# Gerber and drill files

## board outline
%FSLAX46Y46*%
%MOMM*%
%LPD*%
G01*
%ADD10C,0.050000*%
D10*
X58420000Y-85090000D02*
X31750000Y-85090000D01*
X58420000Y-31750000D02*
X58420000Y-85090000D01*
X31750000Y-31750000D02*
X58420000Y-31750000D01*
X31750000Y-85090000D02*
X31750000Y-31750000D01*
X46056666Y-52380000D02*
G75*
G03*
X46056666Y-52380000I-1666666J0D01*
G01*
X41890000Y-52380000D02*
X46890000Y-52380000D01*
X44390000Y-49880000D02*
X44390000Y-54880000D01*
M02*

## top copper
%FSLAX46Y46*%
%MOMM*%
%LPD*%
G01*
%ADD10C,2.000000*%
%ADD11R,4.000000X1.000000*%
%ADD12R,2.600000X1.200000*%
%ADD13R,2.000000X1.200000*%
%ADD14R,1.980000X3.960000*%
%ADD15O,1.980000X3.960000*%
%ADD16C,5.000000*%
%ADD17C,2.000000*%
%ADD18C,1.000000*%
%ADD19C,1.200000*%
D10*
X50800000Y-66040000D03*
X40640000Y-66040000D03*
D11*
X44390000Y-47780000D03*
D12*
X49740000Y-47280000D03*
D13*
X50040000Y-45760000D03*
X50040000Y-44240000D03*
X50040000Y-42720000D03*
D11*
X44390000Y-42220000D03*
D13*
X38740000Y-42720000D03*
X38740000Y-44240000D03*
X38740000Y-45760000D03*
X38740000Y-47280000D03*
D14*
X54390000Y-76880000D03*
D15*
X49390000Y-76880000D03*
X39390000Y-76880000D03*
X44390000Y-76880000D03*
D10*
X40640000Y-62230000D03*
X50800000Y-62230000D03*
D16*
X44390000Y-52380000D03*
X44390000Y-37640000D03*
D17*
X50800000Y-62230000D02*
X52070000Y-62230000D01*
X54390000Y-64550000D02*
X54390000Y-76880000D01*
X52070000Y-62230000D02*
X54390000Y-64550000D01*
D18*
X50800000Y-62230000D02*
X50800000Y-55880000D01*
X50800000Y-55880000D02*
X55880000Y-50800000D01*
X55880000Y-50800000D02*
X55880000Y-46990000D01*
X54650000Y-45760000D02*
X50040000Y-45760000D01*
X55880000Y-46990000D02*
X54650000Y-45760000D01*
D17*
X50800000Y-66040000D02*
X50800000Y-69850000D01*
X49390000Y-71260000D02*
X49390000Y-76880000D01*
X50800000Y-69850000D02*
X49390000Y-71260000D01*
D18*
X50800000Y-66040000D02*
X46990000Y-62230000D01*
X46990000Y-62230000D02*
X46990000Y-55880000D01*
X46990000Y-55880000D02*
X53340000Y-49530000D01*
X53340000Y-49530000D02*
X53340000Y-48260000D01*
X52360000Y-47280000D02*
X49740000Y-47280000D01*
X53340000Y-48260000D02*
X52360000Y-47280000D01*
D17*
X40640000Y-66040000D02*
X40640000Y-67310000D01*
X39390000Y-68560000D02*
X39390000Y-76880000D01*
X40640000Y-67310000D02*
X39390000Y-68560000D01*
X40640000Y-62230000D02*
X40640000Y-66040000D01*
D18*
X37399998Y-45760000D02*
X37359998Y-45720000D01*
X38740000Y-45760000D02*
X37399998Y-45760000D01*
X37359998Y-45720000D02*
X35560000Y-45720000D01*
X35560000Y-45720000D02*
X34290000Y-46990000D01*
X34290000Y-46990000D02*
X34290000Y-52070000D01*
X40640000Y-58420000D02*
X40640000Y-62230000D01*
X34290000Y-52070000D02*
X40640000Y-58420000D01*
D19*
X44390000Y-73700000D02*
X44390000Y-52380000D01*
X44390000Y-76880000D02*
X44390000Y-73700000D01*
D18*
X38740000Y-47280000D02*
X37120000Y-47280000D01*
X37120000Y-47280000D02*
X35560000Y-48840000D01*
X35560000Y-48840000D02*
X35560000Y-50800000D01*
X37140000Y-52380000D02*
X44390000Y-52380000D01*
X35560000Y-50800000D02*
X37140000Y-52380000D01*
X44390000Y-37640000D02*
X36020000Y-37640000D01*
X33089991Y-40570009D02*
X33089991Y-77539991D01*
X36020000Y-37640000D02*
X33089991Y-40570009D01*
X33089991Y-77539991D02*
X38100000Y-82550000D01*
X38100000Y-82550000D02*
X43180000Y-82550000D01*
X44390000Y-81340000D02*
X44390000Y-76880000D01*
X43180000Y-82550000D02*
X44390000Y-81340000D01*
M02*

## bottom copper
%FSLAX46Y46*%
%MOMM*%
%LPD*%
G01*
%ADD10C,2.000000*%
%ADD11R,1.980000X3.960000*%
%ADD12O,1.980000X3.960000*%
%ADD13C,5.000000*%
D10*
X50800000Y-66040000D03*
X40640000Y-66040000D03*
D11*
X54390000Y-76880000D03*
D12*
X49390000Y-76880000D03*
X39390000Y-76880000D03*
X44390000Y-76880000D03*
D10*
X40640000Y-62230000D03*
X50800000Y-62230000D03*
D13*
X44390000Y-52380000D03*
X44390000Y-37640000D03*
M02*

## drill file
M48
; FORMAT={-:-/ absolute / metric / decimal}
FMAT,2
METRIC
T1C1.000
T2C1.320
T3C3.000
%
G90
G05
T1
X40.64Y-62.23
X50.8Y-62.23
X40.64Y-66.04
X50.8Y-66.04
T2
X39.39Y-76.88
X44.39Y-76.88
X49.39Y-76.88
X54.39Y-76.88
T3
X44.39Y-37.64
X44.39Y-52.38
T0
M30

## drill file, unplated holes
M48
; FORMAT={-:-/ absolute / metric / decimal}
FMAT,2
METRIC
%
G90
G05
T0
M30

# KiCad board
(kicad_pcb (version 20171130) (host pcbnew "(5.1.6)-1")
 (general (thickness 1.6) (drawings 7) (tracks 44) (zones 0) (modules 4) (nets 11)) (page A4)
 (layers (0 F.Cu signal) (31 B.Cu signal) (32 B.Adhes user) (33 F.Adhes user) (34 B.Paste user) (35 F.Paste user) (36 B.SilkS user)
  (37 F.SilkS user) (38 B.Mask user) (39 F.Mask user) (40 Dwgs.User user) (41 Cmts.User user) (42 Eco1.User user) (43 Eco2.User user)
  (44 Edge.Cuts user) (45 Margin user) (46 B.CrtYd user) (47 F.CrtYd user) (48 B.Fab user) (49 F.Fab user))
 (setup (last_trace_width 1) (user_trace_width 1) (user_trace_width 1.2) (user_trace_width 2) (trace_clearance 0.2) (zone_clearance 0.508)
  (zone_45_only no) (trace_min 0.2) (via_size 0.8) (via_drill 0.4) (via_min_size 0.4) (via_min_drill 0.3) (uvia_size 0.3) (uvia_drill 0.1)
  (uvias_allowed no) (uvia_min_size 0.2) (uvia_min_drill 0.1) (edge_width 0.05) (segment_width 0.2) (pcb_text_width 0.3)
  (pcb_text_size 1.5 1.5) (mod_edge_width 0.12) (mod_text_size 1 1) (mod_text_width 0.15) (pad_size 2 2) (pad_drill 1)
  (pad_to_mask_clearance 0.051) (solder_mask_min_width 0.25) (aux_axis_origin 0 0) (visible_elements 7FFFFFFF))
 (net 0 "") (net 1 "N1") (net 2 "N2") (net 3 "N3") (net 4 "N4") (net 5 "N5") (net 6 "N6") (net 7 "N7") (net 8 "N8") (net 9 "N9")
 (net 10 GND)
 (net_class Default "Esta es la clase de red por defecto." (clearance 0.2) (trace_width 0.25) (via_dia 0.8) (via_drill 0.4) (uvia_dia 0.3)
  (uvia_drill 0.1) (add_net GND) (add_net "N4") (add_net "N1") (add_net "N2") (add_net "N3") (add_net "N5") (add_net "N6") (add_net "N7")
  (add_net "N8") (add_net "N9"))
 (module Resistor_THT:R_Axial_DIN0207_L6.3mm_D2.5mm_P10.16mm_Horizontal (layer F.Cu) (at 50.8 66.04 180)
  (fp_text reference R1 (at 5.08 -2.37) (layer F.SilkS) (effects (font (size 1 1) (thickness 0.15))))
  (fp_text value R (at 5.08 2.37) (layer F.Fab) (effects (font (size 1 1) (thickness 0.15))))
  (pad 1 thru_hole circle (at 0 0 180) (size 2 2) (drill 1) (layers *.Cu *.Mask) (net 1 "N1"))
  (pad 2 thru_hole circle (at 10.16 0 180) (size 2 2) (drill 1) (layers *.Cu *.Mask) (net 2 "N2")))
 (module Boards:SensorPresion (layer F.Cu) (at 44.39 47.78)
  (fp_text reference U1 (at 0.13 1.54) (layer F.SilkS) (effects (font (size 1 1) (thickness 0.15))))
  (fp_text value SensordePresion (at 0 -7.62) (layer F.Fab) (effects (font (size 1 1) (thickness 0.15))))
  (pad 10 smd rect (at 0 0) (size 4 1) (layers F.Cu F.Paste F.Mask) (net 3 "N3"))
  (pad 1 smd rect (at 5.35 -0.5) (size 2.6 1.2) (layers F.Cu F.Paste F.Mask) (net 1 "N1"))
  (pad 2 smd rect (at 5.65 -2.02) (size 2 1.2) (layers F.Cu F.Paste F.Mask) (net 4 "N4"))
  (pad 3 smd rect (at 5.65 -3.54) (size 2 1.2) (layers F.Cu F.Paste F.Mask) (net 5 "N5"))
  (pad 4 smd rect (at 5.65 -5.06) (size 2 1.2) (layers F.Cu F.Paste F.Mask) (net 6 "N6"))
  (pad 5 smd rect (at 0 -5.56) (size 4 1) (layers F.Cu F.Paste F.Mask) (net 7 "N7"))
  (pad 6 smd rect (at -5.65 -5.06) (size 2 1.2) (layers F.Cu F.Paste F.Mask) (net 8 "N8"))
  (pad 7 smd rect (at -5.65 -3.54) (size 2 1.2) (layers F.Cu F.Paste F.Mask) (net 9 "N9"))
  (pad 8 smd rect (at -5.65 -2.02) (size 2 1.2) (layers F.Cu F.Paste F.Mask) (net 2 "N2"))
  (pad 9 smd rect (at -5.65 -0.5) (size 2 1.2) (layers F.Cu F.Paste F.Mask) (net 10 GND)))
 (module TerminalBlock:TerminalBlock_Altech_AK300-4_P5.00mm (layer F.Cu) (at 54.39 76.88 180)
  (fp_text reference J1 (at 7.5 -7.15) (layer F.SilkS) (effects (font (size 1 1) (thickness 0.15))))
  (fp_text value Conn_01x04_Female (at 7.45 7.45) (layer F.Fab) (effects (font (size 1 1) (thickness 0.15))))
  (pad 1 thru_hole rect (at 0 0 180) (size 1.98 3.96) (drill 1.32) (layers *.Cu *.Mask) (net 4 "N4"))
  (pad 2 thru_hole oval (at 5 0 180) (size 1.98 3.96) (drill 1.32) (layers *.Cu *.Mask) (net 1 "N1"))
  (pad 4 thru_hole oval (at 15 0 180) (size 1.98 3.96) (drill 1.32) (layers *.Cu *.Mask) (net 2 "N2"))
  (pad 3 thru_hole oval (at 10 0 180) (size 1.98 3.96) (drill 1.32) (layers *.Cu *.Mask) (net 10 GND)))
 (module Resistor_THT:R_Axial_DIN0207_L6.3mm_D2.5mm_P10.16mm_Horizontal (layer F.Cu) (at 50.8 62.23 180)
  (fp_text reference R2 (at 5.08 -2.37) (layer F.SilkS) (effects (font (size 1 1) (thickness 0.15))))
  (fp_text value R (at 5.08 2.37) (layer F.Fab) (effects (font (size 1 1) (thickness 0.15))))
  (pad 2 thru_hole circle (at 10.16 0 180) (size 2 2) (drill 1) (layers *.Cu *.Mask) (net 2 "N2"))
  (pad 1 thru_hole circle (at 0 0 180) (size 2 2) (drill 1) (layers *.Cu *.Mask) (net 4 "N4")))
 (gr_line (start 58.42 85.09) (end 31.75 85.09) (layer Edge.Cuts) (width 0.05))
 (gr_line (start 58.42 31.75) (end 58.42 85.09) (layer Edge.Cuts) (width 0.05))
 (gr_line (start 31.75 31.75) (end 58.42 31.75) (layer Edge.Cuts) (width 0.05))
 (gr_line (start 31.75 85.09) (end 31.75 31.75) (layer Edge.Cuts) (width 0.05))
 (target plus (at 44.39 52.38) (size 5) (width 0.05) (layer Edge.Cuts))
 (segment (start 50.8 62.23) (end 52.07 62.23) (width 2) (layer F.Cu) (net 4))
 (segment (start 54.39 64.55) (end 54.39 76.88) (width 2) (layer F.Cu) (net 4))
 (segment (start 52.07 62.23) (end 54.39 64.55) (width 2) (layer F.Cu) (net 4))
 (segment (start 50.8 62.23) (end 50.8 55.88) (width 1) (layer F.Cu) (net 4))
 (segment (start 50.8 55.88) (end 55.88 50.8) (width 1) (layer F.Cu) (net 4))
 (segment (start 55.88 50.8) (end 55.88 46.99) (width 1) (layer F.Cu) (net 4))
 (segment (start 54.65 45.76) (end 50.04 45.76) (width 1) (layer F.Cu) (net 4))
 (segment (start 55.88 46.99) (end 54.65 45.76) (width 1) (layer F.Cu) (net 4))
 (segment (start 50.8 66.04) (end 50.8 69.85) (width 2) (layer F.Cu) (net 1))
 (segment (start 49.39 71.26) (end 49.39 76.88) (width 2) (layer F.Cu) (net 1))
 (segment (start 50.8 69.85) (end 49.39 71.26) (width 2) (layer F.Cu) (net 1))
 (segment (start 50.8 66.04) (end 46.99 62.23) (width 1) (layer F.Cu) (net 1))
 (segment (start 46.99 62.23) (end 46.99 55.88) (width 1) (layer F.Cu) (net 1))
 (segment (start 46.99 55.88) (end 53.34 49.53) (width 1) (layer F.Cu) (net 1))
 (segment (start 53.34 49.53) (end 53.34 48.26) (width 1) (layer F.Cu) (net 1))
 (segment (start 52.36 47.28) (end 49.74 47.28) (width 1) (layer F.Cu) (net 1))
 (segment (start 53.34 48.26) (end 52.36 47.28) (width 1) (layer F.Cu) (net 1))
 (segment (start 40.64 66.04) (end 40.64 67.31) (width 2) (layer F.Cu) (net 2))
 (segment (start 39.39 68.56) (end 39.39 76.88) (width 2) (layer F.Cu) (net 2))
 (segment (start 40.64 67.31) (end 39.39 68.56) (width 2) (layer F.Cu) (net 2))
 (segment (start 40.64 62.23) (end 40.64 66.04) (width 2) (layer F.Cu) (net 2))
 (segment (start 37.399998 45.76) (end 37.359998 45.72) (width 1) (layer F.Cu) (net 2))
 (segment (start 38.74 45.76) (end 37.399998 45.76) (width 1) (layer F.Cu) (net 2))
 (segment (start 37.359998 45.72) (end 35.56 45.72) (width 1) (layer F.Cu) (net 2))
 (segment (start 35.56 45.72) (end 34.29 46.99) (width 1) (layer F.Cu) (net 2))
 (segment (start 34.29 46.99) (end 34.29 52.07) (width 1) (layer F.Cu) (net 2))
 (segment (start 40.64 58.42) (end 40.64 62.23) (width 1) (layer F.Cu) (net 2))
 (segment (start 34.29 52.07) (end 40.64 58.42) (width 1) (layer F.Cu) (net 2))
 (via (at 44.39 52.38) (size 5) (drill 3) (layers F.Cu B.Cu) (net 10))
 (segment (start 44.39 73.7) (end 44.39 52.38) (width 1.2) (layer F.Cu) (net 10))
 (segment (start 44.39 76.88) (end 44.39 73.7) (width 1.2) (layer F.Cu) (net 10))
 (via (at 44.39 37.64) (size 5) (drill 3) (layers F.Cu B.Cu) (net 10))
 (segment (start 38.74 47.28) (end 37.12 47.28) (width 1) (layer F.Cu) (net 10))
 (segment (start 37.12 47.28) (end 35.56 48.84) (width 1) (layer F.Cu) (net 10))
 (segment (start 35.56 48.84) (end 35.56 50.8) (width 1) (layer F.Cu) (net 10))
 (segment (start 37.14 52.38) (end 44.39 52.38) (width 1) (layer F.Cu) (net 10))
 (segment (start 35.56 50.8) (end 37.14 52.38) (width 1) (layer F.Cu) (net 10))
 (segment (start 44.39 37.64) (end 36.02 37.64) (width 1) (layer F.Cu) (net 10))
 (segment (start 33.089991 40.570009) (end 33.089991 77.539991) (width 1) (layer F.Cu) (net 10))
 (segment (start 36.02 37.64) (end 33.089991 40.570009) (width 1) (layer F.Cu) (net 10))
 (segment (start 33.089991 77.539991) (end 38.1 82.55) (width 1) (layer F.Cu) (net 10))
 (segment (start 38.1 82.55) (end 43.18 82.55) (width 1) (layer F.Cu) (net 10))
 (segment (start 44.39 81.34) (end 44.39 76.88) (width 1) (layer F.Cu) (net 10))
 (segment (start 43.18 82.55) (end 44.39 81.34) (width 1) (layer F.Cu) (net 10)))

